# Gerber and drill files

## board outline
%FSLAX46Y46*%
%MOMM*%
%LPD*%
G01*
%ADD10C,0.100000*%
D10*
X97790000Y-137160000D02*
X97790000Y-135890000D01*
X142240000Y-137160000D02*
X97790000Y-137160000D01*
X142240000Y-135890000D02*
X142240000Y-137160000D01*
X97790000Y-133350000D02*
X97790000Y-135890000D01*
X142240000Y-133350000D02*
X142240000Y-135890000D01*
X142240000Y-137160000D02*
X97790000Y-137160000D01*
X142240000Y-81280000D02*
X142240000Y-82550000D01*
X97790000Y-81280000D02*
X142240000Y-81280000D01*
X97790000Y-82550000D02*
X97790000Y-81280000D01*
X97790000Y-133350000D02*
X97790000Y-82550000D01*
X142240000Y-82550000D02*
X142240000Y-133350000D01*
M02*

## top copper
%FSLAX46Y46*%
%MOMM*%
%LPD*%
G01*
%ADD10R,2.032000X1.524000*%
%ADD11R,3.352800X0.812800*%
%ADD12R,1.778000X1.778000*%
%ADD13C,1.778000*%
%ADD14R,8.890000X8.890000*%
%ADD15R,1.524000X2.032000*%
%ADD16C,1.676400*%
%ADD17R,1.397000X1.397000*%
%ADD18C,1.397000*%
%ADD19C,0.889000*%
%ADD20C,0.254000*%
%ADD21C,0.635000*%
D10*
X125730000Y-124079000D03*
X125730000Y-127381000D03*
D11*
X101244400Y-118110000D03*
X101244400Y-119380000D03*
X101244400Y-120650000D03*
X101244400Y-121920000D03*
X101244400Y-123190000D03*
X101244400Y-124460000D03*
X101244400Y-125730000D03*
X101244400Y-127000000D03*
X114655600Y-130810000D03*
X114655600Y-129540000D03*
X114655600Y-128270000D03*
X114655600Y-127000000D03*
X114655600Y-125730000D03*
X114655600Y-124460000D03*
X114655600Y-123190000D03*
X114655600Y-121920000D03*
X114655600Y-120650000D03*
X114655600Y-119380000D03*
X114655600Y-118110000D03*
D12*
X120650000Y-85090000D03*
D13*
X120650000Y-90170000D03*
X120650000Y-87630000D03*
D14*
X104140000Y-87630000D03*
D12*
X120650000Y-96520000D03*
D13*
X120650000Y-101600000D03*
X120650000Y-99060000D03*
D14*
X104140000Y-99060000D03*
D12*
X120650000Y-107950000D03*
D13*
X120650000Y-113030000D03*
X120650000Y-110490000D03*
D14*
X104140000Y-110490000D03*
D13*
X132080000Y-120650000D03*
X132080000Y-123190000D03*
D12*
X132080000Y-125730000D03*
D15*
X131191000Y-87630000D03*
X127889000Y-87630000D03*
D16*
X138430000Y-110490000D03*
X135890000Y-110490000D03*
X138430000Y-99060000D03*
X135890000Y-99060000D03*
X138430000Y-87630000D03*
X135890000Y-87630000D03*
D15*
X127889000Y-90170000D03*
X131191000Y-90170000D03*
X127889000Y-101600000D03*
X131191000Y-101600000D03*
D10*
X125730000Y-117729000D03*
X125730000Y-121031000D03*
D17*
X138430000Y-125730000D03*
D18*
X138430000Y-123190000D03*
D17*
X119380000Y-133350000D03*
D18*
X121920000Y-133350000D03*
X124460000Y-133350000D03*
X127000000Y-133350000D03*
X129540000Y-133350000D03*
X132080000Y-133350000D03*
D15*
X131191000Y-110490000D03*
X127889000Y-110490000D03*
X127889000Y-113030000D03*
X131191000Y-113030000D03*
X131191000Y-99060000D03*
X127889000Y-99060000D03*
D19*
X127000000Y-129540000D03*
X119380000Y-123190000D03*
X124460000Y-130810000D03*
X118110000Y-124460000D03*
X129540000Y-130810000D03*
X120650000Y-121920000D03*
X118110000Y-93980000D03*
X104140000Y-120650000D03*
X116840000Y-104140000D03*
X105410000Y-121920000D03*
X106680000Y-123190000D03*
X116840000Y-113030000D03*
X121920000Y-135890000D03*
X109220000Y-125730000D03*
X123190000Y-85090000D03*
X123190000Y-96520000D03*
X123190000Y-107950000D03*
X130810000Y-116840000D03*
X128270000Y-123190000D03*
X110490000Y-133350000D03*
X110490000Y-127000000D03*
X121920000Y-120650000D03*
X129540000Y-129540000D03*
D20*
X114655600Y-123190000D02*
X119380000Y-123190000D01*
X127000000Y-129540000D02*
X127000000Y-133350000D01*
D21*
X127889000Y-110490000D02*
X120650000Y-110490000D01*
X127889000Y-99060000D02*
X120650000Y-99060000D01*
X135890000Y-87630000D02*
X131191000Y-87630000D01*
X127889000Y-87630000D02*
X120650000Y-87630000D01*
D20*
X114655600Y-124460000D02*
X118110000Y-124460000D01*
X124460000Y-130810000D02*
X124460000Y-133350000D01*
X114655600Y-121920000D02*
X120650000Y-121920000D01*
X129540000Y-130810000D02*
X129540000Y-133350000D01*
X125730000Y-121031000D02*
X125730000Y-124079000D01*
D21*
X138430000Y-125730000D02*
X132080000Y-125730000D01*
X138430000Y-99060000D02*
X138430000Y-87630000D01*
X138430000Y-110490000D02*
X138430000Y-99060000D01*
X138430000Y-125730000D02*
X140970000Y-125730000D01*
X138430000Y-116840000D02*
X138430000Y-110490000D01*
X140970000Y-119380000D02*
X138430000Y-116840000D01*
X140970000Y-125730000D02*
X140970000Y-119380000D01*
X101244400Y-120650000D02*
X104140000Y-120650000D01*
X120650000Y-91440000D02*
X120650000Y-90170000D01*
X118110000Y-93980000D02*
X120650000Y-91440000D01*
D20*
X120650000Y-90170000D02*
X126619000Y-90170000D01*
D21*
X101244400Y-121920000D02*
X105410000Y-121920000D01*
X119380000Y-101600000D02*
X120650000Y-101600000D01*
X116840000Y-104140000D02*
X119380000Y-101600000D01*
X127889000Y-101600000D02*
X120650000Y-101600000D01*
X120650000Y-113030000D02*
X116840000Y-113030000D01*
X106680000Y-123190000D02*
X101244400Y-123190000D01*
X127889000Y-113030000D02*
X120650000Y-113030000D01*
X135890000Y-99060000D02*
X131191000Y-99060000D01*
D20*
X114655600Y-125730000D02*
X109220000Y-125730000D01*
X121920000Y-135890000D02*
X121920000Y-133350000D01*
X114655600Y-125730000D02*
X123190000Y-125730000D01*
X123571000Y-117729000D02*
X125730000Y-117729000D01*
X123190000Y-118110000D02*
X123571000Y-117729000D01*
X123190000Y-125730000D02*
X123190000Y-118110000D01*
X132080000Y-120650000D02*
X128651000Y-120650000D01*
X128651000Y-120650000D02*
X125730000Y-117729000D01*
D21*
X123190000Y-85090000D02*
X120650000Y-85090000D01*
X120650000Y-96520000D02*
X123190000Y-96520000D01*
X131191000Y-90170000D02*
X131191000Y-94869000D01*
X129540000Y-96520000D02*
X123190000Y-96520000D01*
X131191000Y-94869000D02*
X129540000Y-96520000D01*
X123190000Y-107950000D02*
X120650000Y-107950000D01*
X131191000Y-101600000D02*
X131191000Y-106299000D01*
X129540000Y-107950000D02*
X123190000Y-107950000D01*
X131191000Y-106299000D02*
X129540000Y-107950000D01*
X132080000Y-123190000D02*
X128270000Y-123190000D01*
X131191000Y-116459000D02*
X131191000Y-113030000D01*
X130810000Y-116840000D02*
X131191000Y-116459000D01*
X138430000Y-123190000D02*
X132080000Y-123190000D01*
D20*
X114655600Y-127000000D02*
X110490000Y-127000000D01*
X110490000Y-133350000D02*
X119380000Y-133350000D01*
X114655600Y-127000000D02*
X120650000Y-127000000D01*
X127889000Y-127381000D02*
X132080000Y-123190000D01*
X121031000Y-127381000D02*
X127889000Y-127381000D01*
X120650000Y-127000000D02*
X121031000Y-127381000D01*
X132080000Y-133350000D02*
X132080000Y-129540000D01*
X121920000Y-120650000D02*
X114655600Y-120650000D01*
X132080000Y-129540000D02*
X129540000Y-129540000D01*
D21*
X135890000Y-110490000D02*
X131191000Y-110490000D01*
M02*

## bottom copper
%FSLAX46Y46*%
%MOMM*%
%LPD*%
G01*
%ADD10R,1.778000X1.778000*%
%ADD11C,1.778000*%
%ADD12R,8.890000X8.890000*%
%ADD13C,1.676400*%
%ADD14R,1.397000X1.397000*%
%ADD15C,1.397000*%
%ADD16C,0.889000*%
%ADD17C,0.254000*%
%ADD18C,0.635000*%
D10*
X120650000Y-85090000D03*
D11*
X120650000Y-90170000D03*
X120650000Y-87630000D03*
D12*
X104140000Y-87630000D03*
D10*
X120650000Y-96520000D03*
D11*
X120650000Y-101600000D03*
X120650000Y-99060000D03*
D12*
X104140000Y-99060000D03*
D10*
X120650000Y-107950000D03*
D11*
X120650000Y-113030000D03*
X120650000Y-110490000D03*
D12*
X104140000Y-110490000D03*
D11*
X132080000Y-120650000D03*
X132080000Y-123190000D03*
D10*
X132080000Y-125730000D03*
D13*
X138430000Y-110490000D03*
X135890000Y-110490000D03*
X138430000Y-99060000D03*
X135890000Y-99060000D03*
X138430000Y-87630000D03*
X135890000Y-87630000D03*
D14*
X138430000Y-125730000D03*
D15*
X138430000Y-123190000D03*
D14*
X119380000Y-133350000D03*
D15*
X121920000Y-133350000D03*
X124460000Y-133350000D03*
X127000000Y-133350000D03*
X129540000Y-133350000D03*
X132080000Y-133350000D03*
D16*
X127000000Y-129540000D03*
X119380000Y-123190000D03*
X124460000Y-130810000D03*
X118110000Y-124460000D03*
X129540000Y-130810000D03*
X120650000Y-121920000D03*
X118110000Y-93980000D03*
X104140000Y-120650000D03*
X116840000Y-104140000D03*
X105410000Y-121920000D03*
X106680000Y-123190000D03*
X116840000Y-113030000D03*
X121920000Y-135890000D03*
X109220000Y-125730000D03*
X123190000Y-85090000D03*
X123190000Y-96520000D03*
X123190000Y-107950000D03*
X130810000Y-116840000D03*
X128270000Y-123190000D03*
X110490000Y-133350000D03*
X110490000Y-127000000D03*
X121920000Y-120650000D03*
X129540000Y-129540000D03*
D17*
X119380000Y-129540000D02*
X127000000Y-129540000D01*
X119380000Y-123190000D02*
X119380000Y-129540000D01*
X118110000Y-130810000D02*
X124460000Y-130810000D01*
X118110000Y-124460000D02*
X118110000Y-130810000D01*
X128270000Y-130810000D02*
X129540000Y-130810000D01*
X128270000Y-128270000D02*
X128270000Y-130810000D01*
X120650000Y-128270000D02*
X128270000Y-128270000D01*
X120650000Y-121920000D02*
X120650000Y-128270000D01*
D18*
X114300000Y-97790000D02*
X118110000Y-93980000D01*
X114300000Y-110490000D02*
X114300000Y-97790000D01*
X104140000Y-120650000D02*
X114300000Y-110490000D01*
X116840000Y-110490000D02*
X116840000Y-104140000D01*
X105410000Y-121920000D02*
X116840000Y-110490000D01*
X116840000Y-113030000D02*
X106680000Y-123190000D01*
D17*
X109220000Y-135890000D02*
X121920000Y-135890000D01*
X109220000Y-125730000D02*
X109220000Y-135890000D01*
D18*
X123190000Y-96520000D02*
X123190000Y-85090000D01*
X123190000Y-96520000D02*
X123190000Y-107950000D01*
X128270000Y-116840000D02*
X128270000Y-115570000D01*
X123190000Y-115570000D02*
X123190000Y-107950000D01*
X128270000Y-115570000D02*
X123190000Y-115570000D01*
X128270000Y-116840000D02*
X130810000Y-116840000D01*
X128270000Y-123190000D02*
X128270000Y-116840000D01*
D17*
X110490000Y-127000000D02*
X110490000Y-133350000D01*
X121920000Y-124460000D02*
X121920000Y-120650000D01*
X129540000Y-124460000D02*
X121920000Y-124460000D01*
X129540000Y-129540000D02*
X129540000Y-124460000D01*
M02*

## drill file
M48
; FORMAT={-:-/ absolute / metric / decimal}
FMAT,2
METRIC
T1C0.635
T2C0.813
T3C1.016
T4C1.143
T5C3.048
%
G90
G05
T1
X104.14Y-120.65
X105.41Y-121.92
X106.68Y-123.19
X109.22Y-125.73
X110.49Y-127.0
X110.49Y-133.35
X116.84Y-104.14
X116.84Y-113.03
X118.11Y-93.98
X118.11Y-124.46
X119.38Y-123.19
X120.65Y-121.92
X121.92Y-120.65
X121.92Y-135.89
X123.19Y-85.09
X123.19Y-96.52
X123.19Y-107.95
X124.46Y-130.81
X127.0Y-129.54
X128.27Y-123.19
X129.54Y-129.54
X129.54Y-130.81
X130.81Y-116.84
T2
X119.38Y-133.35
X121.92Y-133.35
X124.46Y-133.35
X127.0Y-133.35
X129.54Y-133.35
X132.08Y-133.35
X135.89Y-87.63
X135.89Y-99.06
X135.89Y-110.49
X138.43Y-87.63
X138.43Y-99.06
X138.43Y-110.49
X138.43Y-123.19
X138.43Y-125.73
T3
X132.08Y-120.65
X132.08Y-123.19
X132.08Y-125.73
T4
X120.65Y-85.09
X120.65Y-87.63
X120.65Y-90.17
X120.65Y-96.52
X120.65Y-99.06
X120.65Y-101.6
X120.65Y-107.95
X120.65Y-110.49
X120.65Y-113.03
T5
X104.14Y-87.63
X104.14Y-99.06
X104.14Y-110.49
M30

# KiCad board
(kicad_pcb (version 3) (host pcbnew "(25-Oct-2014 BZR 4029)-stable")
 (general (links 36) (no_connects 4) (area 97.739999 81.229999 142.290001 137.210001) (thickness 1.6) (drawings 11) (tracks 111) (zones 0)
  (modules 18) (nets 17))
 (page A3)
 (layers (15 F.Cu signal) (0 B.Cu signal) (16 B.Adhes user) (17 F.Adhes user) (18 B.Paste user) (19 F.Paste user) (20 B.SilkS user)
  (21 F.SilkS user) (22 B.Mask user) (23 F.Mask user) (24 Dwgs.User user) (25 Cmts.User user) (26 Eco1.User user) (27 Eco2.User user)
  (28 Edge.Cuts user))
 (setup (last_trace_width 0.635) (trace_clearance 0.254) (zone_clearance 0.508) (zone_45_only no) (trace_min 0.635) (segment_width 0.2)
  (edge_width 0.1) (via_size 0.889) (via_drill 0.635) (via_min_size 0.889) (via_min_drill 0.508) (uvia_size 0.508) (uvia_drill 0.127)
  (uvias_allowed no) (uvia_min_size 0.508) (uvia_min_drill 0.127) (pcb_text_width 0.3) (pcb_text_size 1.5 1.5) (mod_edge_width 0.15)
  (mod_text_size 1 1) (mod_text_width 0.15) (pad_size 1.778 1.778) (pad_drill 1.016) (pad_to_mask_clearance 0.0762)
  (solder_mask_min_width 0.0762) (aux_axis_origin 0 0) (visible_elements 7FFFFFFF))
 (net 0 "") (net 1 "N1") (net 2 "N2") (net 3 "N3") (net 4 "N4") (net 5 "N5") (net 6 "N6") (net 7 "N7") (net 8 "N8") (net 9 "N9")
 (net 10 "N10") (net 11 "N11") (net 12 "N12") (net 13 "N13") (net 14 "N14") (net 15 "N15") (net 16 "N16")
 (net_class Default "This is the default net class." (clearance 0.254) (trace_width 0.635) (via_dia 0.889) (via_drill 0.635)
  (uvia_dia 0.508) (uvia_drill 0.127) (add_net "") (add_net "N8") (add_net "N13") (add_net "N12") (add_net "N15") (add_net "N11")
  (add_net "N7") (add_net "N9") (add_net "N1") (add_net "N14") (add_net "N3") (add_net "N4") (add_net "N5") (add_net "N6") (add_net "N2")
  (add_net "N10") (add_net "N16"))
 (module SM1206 (layer F.Cu) (at 125.73 125.73 270)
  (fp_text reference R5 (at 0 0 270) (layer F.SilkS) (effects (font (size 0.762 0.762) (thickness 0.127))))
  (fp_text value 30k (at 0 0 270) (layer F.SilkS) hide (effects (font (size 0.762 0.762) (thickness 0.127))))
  (pad 1 smd rect (at -1.651 0 270) (size 1.524 2.032) (layers F.Cu F.Paste F.Mask) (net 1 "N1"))
  (pad 2 smd rect (at 1.651 0 270) (size 1.524 2.032) (layers F.Cu F.Paste F.Mask) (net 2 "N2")))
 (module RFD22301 (layer F.Cu) (at 106.68 125.73)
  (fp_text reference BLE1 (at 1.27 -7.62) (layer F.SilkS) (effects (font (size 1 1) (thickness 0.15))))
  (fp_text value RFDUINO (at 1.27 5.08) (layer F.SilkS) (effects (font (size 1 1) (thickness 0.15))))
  (pad 1 smd rect (at -5.4356 -7.62) (size 3.3528 0.8128) (layers F.Cu F.Paste F.Mask))
  (pad 2 smd rect (at -5.4356 -6.35) (size 3.3528 0.8128) (layers F.Cu F.Paste F.Mask))
  (pad 3 smd rect (at -5.4356 -5.08) (size 3.3528 0.8128) (layers F.Cu F.Paste F.Mask) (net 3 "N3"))
  (pad 4 smd rect (at -5.4356 -3.81) (size 3.3528 0.8128) (layers F.Cu F.Paste F.Mask) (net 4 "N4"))
  (pad 5 smd rect (at -5.4356 -2.54) (size 3.3528 0.8128) (layers F.Cu F.Paste F.Mask) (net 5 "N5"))
  (pad 6 smd rect (at -5.4356 -1.27) (size 3.3528 0.8128) (layers F.Cu F.Paste F.Mask) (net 1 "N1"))
  (pad 7 smd rect (at -5.4356 0) (size 3.3528 0.8128) (layers F.Cu F.Paste F.Mask))
  (pad 8 smd rect (at -5.4356 1.27) (size 3.3528 0.8128) (layers F.Cu F.Paste F.Mask))
  (pad 9 smd rect (at 7.9756 5.08) (size 3.3528 0.8128) (layers F.Cu F.Paste F.Mask))
  (pad 10 smd rect (at 7.9756 3.81) (size 3.3528 0.8128) (layers F.Cu F.Paste F.Mask))
  (pad 11 smd rect (at 7.9756 2.54) (size 3.3528 0.8128) (layers F.Cu F.Paste F.Mask))
  (pad 12 smd rect (at 7.9756 1.27) (size 3.3528 0.8128) (layers F.Cu F.Paste F.Mask) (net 2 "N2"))
  (pad 13 smd rect (at 7.9756 0) (size 3.3528 0.8128) (layers F.Cu F.Paste F.Mask) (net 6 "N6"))
  (pad 14 smd rect (at 7.9756 -1.27) (size 3.3528 0.8128) (layers F.Cu F.Paste F.Mask) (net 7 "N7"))
  (pad 15 smd rect (at 7.9756 -2.54) (size 3.3528 0.8128) (layers F.Cu F.Paste F.Mask) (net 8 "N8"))
  (pad 16 smd rect (at 7.9756 -3.81) (size 3.3528 0.8128) (layers F.Cu F.Paste F.Mask) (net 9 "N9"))
  (pad 17 smd rect (at 7.9756 -5.08) (size 3.3528 0.8128) (layers F.Cu F.Paste F.Mask) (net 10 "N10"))
  (pad 18 smd rect (at 7.9756 -6.35) (size 3.3528 0.8128) (layers F.Cu F.Paste F.Mask))
  (pad 19 smd rect (at 7.9756 -7.62) (size 3.3528 0.8128) (layers F.Cu F.Paste F.Mask)))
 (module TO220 (layer F.Cu) (at 120.65 87.63 180)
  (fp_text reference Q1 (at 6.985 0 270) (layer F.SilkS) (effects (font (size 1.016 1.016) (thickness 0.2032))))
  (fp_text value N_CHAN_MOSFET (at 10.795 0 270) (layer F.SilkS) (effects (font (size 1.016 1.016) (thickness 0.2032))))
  (pad 1 thru_hole rect (at 0 2.54 180) (size 1.778 1.778) (drill 1.143) (layers *.Cu *.Mask F.SilkS) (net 2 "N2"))
  (pad 2 thru_hole circle (at 0 -2.54 180) (size 1.778 1.778) (drill 1.143) (layers *.Cu *.Mask F.SilkS) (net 3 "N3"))
  (pad 3 thru_hole circle (at 0 0 180) (size 1.778 1.778) (drill 1.143) (layers *.Cu *.Mask F.SilkS) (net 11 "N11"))
  (pad 4 thru_hole rect (at 16.51 0 180) (size 8.89 8.89) (drill 3.048) (layers *.Cu *.SilkS *.Mask)))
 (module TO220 (layer F.Cu) (at 120.65 99.06 180)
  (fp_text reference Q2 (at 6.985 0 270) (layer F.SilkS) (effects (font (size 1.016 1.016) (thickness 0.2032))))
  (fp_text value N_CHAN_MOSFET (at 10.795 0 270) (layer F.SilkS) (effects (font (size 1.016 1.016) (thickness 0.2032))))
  (pad 1 thru_hole rect (at 0 2.54 180) (size 1.778 1.778) (drill 1.143) (layers *.Cu *.Mask F.SilkS) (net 2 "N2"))
  (pad 2 thru_hole circle (at 0 -2.54 180) (size 1.778 1.778) (drill 1.143) (layers *.Cu *.Mask F.SilkS) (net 4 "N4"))
  (pad 3 thru_hole circle (at 0 0 180) (size 1.778 1.778) (drill 1.143) (layers *.Cu *.Mask F.SilkS) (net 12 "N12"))
  (pad 4 thru_hole rect (at 16.51 0 180) (size 8.89 8.89) (drill 3.048) (layers *.Cu *.SilkS *.Mask)))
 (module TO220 (layer F.Cu) (at 120.65 110.49 180)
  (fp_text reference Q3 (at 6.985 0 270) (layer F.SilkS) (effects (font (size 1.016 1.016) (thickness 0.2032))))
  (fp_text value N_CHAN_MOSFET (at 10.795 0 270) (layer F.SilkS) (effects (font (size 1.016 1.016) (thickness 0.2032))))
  (pad 1 thru_hole rect (at 0 2.54 180) (size 1.778 1.778) (drill 1.143) (layers *.Cu *.Mask F.SilkS) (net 2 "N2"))
  (pad 2 thru_hole circle (at 0 -2.54 180) (size 1.778 1.778) (drill 1.143) (layers *.Cu *.Mask F.SilkS) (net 5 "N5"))
  (pad 3 thru_hole circle (at 0 0 180) (size 1.778 1.778) (drill 1.143) (layers *.Cu *.Mask F.SilkS) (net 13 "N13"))
  (pad 4 thru_hole rect (at 16.51 0 180) (size 8.89 8.89) (drill 3.048) (layers *.Cu *.SilkS *.Mask)))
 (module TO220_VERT (layer F.Cu) (at 132.08 123.19)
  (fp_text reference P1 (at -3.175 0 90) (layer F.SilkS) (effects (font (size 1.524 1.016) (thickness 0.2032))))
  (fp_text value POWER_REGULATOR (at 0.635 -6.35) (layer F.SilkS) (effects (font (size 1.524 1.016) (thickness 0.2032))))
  (pad 2 thru_hole circle (at 0 -2.54) (size 1.778 1.778) (drill 1.016) (layers *.Cu *.Mask F.SilkS) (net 6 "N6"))
  (pad 3 thru_hole circle (at 0 0) (size 1.778 1.778) (drill 1.016) (layers *.Cu *.Mask F.SilkS) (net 2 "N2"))
  (pad 1 thru_hole rect (at 0 2.54) (size 1.778 1.778) (drill 1.016) (layers *.Cu *.Mask F.SilkS) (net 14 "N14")))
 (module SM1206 (layer F.Cu) (at 129.54 87.63 180)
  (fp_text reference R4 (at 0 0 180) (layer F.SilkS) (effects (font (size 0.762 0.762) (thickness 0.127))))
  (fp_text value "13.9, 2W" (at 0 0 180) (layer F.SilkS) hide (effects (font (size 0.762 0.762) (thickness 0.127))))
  (pad 1 smd rect (at -1.651 0 180) (size 1.524 2.032) (layers F.Cu F.Paste F.Mask) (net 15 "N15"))
  (pad 2 smd rect (at 1.651 0 180) (size 1.524 2.032) (layers F.Cu F.Paste F.Mask) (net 11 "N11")))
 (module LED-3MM (layer F.Cu) (at 137.16 110.49 180)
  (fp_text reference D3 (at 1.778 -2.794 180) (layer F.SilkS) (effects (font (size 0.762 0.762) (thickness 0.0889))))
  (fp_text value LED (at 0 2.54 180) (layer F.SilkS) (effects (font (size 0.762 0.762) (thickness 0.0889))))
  (pad 1 thru_hole circle (at -1.27 0 180) (size 1.6764 1.6764) (drill 0.8128) (layers *.Cu *.Mask F.SilkS) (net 14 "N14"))
  (pad 2 thru_hole circle (at 1.27 0 180) (size 1.6764 1.6764) (drill 0.8128) (layers *.Cu *.Mask F.SilkS) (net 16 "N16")))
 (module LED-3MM (layer F.Cu) (at 137.16 99.06 180)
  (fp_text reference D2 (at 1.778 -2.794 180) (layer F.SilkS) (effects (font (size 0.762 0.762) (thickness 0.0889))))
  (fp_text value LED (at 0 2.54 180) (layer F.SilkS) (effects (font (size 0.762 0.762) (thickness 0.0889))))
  (pad 1 thru_hole circle (at -1.27 0 180) (size 1.6764 1.6764) (drill 0.8128) (layers *.Cu *.Mask F.SilkS) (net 14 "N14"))
  (pad 2 thru_hole circle (at 1.27 0 180) (size 1.6764 1.6764) (drill 0.8128) (layers *.Cu *.Mask F.SilkS) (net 5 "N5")))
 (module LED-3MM (layer F.Cu) (at 137.16 87.63 180)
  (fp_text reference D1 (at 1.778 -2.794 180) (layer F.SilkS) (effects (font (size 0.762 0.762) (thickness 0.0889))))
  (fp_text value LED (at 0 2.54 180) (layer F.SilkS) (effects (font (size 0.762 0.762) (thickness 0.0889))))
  (pad 1 thru_hole circle (at -1.27 0 180) (size 1.6764 1.6764) (drill 0.8128) (layers *.Cu *.Mask F.SilkS) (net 14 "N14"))
  (pad 2 thru_hole circle (at 1.27 0 180) (size 1.6764 1.6764) (drill 0.8128) (layers *.Cu *.Mask F.SilkS) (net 15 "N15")))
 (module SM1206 (layer F.Cu) (at 129.54 90.17)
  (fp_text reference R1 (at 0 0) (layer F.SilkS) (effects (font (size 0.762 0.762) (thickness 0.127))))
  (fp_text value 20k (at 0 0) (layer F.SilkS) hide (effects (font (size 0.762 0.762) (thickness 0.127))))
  (pad 1 smd rect (at -1.651 0) (size 1.524 2.032) (layers F.Cu F.Paste F.Mask) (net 3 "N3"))
  (pad 2 smd rect (at 1.651 0) (size 1.524 2.032) (layers F.Cu F.Paste F.Mask) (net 2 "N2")))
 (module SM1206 (layer F.Cu) (at 129.54 101.6)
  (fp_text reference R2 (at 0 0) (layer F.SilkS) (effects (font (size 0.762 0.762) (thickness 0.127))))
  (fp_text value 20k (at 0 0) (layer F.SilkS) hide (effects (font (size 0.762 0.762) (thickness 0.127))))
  (pad 1 smd rect (at -1.651 0) (size 1.524 2.032) (layers F.Cu F.Paste F.Mask) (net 4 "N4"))
  (pad 2 smd rect (at 1.651 0) (size 1.524 2.032) (layers F.Cu F.Paste F.Mask) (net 2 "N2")))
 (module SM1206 (layer F.Cu) (at 125.73 119.38 270)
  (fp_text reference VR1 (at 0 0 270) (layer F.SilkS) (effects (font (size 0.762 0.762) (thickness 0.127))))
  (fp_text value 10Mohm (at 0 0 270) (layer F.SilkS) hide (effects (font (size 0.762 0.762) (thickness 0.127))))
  (pad 1 smd rect (at -1.651 0 270) (size 1.524 2.032) (layers F.Cu F.Paste F.Mask) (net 6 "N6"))
  (pad 2 smd rect (at 1.651 0 270) (size 1.524 2.032) (layers F.Cu F.Paste F.Mask) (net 1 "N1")))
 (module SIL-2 (layer F.Cu) (at 138.43 124.46 90)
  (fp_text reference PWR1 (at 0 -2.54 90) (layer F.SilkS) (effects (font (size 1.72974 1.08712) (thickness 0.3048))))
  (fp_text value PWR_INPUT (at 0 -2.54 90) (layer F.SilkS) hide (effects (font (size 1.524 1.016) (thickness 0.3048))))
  (pad 1 thru_hole rect (at -1.27 0 90) (size 1.397 1.397) (drill 0.8128) (layers *.Cu *.Mask F.SilkS) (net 14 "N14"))
  (pad 2 thru_hole circle (at 1.27 0 90) (size 1.397 1.397) (drill 0.8128) (layers *.Cu *.Mask F.SilkS) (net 2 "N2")))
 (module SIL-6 (layer F.Cu) (at 125.73 133.35)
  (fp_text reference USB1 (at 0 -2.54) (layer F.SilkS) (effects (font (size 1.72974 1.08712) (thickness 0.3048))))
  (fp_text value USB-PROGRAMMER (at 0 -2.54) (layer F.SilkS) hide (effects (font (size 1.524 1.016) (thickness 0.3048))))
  (pad 1 thru_hole rect (at -6.35 0) (size 1.397 1.397) (drill 0.8128) (layers *.Cu *.Mask F.SilkS) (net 2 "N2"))
  (pad 2 thru_hole circle (at -3.81 0) (size 1.397 1.397) (drill 0.8128) (layers *.Cu *.Mask F.SilkS) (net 6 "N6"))
  (pad 3 thru_hole circle (at -1.27 0) (size 1.397 1.397) (drill 0.8128) (layers *.Cu *.Mask F.SilkS) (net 7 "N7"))
  (pad 4 thru_hole circle (at 1.27 0) (size 1.397 1.397) (drill 0.8128) (layers *.Cu *.Mask F.SilkS) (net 8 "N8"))
  (pad 5 thru_hole circle (at 3.81 0) (size 1.397 1.397) (drill 0.8128) (layers *.Cu *.Mask F.SilkS) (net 9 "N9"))
  (pad 6 thru_hole circle (at 6.35 0) (size 1.397 1.397) (drill 0.8128) (layers *.Cu *.Mask F.SilkS) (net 10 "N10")))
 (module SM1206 (layer F.Cu) (at 129.54 110.49 180)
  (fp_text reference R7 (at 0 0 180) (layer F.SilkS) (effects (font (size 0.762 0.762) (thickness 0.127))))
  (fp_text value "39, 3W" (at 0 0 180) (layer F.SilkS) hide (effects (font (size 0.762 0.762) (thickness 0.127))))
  (pad 1 smd rect (at -1.651 0 180) (size 1.524 2.032) (layers F.Cu F.Paste F.Mask) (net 16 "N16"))
  (pad 2 smd rect (at 1.651 0 180) (size 1.524 2.032) (layers F.Cu F.Paste F.Mask) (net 13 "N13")))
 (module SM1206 (layer F.Cu) (at 129.54 113.03)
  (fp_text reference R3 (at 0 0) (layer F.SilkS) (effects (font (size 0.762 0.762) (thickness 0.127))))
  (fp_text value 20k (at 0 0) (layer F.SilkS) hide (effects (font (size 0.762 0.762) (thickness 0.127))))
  (pad 1 smd rect (at -1.651 0) (size 1.524 2.032) (layers F.Cu F.Paste F.Mask) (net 5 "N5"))
  (pad 2 smd rect (at 1.651 0) (size 1.524 2.032) (layers F.Cu F.Paste F.Mask) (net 2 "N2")))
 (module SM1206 (layer F.Cu) (at 129.54 99.06 180)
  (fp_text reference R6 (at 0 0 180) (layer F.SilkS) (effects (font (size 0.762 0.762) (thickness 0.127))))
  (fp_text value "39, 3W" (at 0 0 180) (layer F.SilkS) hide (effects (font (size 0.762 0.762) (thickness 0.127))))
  (pad 1 smd rect (at -1.651 0 180) (size 1.524 2.032) (layers F.Cu F.Paste F.Mask) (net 5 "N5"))
  (pad 2 smd rect (at 1.651 0 180) (size 1.524 2.032) (layers F.Cu F.Paste F.Mask) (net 12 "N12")))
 (gr_line (start 97.79 137.16) (end 97.79 135.89) (angle 90) (layer Edge.Cuts) (width 0.1))
 (gr_line (start 142.24 137.16) (end 97.79 137.16) (angle 90) (layer Edge.Cuts) (width 0.1))
 (gr_line (start 142.24 135.89) (end 142.24 137.16) (angle 90) (layer Edge.Cuts) (width 0.1))
 (gr_line (start 97.79 133.35) (end 97.79 135.89) (angle 90) (layer Edge.Cuts) (width 0.1))
 (gr_line (start 142.24 133.35) (end 142.24 135.89) (angle 90) (layer Edge.Cuts) (width 0.1))
 (gr_line (start 142.24 137.16) (end 97.79 137.16) (angle 90) (layer Edge.Cuts) (width 0.1))
 (gr_line (start 142.24 81.28) (end 142.24 82.55) (angle 90) (layer Edge.Cuts) (width 0.1))
 (gr_line (start 97.79 81.28) (end 142.24 81.28) (angle 90) (layer Edge.Cuts) (width 0.1))
 (gr_line (start 97.79 82.55) (end 97.79 81.28) (angle 90) (layer Edge.Cuts) (width 0.1))
 (gr_line (start 97.79 133.35) (end 97.79 82.55) (angle 90) (layer Edge.Cuts) (width 0.1))
 (gr_line (start 142.24 82.55) (end 142.24 133.35) (angle 90) (layer Edge.Cuts) (width 0.1))
 (segment (start 114.6556 123.19) (end 119.38 123.19) (width 0.254) (layer F.Cu) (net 8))
 (segment (start 127 129.54) (end 127 133.35) (width 0.254) (layer F.Cu) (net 8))
 (via (at 127 129.54) (size 0.889) (layers F.Cu B.Cu) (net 8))
 (segment (start 119.38 129.54) (end 127 129.54) (width 0.254) (layer B.Cu) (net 8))
 (segment (start 119.38 123.19) (end 119.38 129.54) (width 0.254) (layer B.Cu) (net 8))
 (via (at 119.38 123.19) (size 0.889) (layers F.Cu B.Cu) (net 8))
 (segment (start 127.889 110.49) (end 120.65 110.49) (width 0.635) (layer F.Cu) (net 13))
 (segment (start 127.889 99.06) (end 120.65 99.06) (width 0.635) (layer F.Cu) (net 12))
 (segment (start 135.89 87.63) (end 131.191 87.63) (width 0.635) (layer F.Cu) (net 15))
 (segment (start 127.889 87.63) (end 120.65 87.63) (width 0.635) (layer F.Cu) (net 11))
 (segment (start 114.6556 124.46) (end 118.11 124.46) (width 0.254) (layer F.Cu) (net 7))
 (segment (start 124.46 130.81) (end 124.46 133.35) (width 0.254) (layer F.Cu) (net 7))
 (via (at 124.46 130.81) (size 0.889) (layers F.Cu B.Cu) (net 7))
 (segment (start 118.11 130.81) (end 124.46 130.81) (width 0.254) (layer B.Cu) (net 7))
 (segment (start 118.11 124.46) (end 118.11 130.81) (width 0.254) (layer B.Cu) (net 7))
 (via (at 118.11 124.46) (size 0.889) (layers F.Cu B.Cu) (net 7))
 (segment (start 114.6556 121.92) (end 120.65 121.92) (width 0.254) (layer F.Cu) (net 9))
 (segment (start 129.54 130.81) (end 129.54 133.35) (width 0.254) (layer F.Cu) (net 9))
 (via (at 129.54 130.81) (size 0.889) (layers F.Cu B.Cu) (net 9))
 (segment (start 128.27 130.81) (end 129.54 130.81) (width 0.254) (layer B.Cu) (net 9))
 (segment (start 128.27 128.27) (end 128.27 130.81) (width 0.254) (layer B.Cu) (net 9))
 (segment (start 120.65 128.27) (end 128.27 128.27) (width 0.254) (layer B.Cu) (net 9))
 (segment (start 120.65 121.92) (end 120.65 128.27) (width 0.254) (layer B.Cu) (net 9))
 (via (at 120.65 121.92) (size 0.889) (layers F.Cu B.Cu) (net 9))
 (segment (start 125.73 121.031) (end 125.73 124.079) (width 0.254) (layer F.Cu) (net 1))
 (segment (start 138.43 125.73) (end 132.08 125.73) (width 0.635) (layer F.Cu) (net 14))
 (segment (start 138.43 99.06) (end 138.43 87.63) (width 0.635) (layer F.Cu) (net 14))
 (segment (start 138.43 110.49) (end 138.43 99.06) (width 0.635) (layer F.Cu) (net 14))
 (segment (start 138.43 125.73) (end 140.97 125.73) (width 0.635) (layer F.Cu) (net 14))
 (segment (start 138.43 116.84) (end 138.43 110.49) (width 0.635) (layer F.Cu) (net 14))
 (segment (start 140.97 119.38) (end 138.43 116.84) (width 0.635) (layer F.Cu) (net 14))
 (segment (start 140.97 125.73) (end 140.97 119.38) (width 0.635) (layer F.Cu) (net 14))
 (segment (start 101.2444 120.65) (end 104.14 120.65) (width 0.635) (layer F.Cu) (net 3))
 (segment (start 120.65 91.44) (end 120.65 90.17) (width 0.635) (layer F.Cu) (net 3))
 (segment (start 118.11 93.98) (end 120.65 91.44) (width 0.635) (layer F.Cu) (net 3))
 (via (at 118.11 93.98) (size 0.889) (layers F.Cu B.Cu) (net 3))
 (segment (start 114.3 97.79) (end 118.11 93.98) (width 0.635) (layer B.Cu) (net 3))
 (segment (start 114.3 110.49) (end 114.3 97.79) (width 0.635) (layer B.Cu) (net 3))
 (segment (start 104.14 120.65) (end 114.3 110.49) (width 0.635) (layer B.Cu) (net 3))
 (via (at 104.14 120.65) (size 0.889) (layers F.Cu B.Cu) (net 3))
 (segment (start 120.65 90.17) (end 126.619 90.17) (width 0.254) (layer F.Cu) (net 3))
 (segment (start 101.2444 121.92) (end 105.41 121.92) (width 0.635) (layer F.Cu) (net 4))
 (segment (start 119.38 101.6) (end 120.65 101.6) (width 0.635) (layer F.Cu) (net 4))
 (segment (start 116.84 104.14) (end 119.38 101.6) (width 0.635) (layer F.Cu) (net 4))
 (via (at 116.84 104.14) (size 0.889) (layers F.Cu B.Cu) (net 4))
 (segment (start 116.84 110.49) (end 116.84 104.14) (width 0.635) (layer B.Cu) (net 4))
 (segment (start 105.41 121.92) (end 116.84 110.49) (width 0.635) (layer B.Cu) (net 4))
 (via (at 105.41 121.92) (size 0.889) (layers F.Cu B.Cu) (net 4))
 (segment (start 127.889 101.6) (end 120.65 101.6) (width 0.635) (layer F.Cu) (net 4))
 (segment (start 120.65 113.03) (end 116.84 113.03) (width 0.635) (layer F.Cu) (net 5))
 (segment (start 106.68 123.19) (end 101.2444 123.19) (width 0.635) (layer F.Cu) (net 5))
 (via (at 106.68 123.19) (size 0.889) (layers F.Cu B.Cu) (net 5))
 (segment (start 116.84 113.03) (end 106.68 123.19) (width 0.635) (layer B.Cu) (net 5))
 (via (at 116.84 113.03) (size 0.889) (layers F.Cu B.Cu) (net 5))
 (segment (start 127.889 113.03) (end 120.65 113.03) (width 0.635) (layer F.Cu) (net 5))
 (segment (start 135.89 99.06) (end 131.191 99.06) (width 0.635) (layer F.Cu) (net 5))
 (segment (start 114.6556 125.73) (end 109.22 125.73) (width 0.254) (layer F.Cu) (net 6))
 (segment (start 121.92 135.89) (end 121.92 133.35) (width 0.254) (layer F.Cu) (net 6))
 (via (at 121.92 135.89) (size 0.889) (layers F.Cu B.Cu) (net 6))
 (segment (start 109.22 135.89) (end 121.92 135.89) (width 0.254) (layer B.Cu) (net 6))
 (segment (start 109.22 125.73) (end 109.22 135.89) (width 0.254) (layer B.Cu) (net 6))
 (via (at 109.22 125.73) (size 0.889) (layers F.Cu B.Cu) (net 6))
 (segment (start 114.6556 125.73) (end 123.19 125.73) (width 0.254) (layer F.Cu) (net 6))
 (segment (start 123.571 117.729) (end 125.73 117.729) (width 0.254) (layer F.Cu) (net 6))
 (segment (start 123.19 118.11) (end 123.571 117.729) (width 0.254) (layer F.Cu) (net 6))
 (segment (start 123.19 125.73) (end 123.19 118.11) (width 0.254) (layer F.Cu) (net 6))
 (segment (start 132.08 120.65) (end 128.651 120.65) (width 0.254) (layer F.Cu) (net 6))
 (segment (start 128.651 120.65) (end 125.73 117.729) (width 0.254) (layer F.Cu) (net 6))
 (segment (start 123.19 96.52) (end 123.19 85.09) (width 0.635) (layer B.Cu) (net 2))
 (segment (start 123.19 85.09) (end 120.65 85.09) (width 0.635) (layer F.Cu) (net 2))
 (via (at 123.19 85.09) (size 0.889) (layers F.Cu B.Cu) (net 2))
 (segment (start 120.65 96.52) (end 123.19 96.52) (width 0.635) (layer F.Cu) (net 2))
 (segment (start 131.191 90.17) (end 131.191 94.869) (width 0.635) (layer F.Cu) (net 2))
 (segment (start 123.19 96.52) (end 123.19 107.95) (width 0.635) (layer B.Cu) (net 2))
 (via (at 123.19 96.52) (size 0.889) (layers F.Cu B.Cu) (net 2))
 (segment (start 129.54 96.52) (end 123.19 96.52) (width 0.635) (layer F.Cu) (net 2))
 (segment (start 131.191 94.869) (end 129.54 96.52) (width 0.635) (layer F.Cu) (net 2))
 (segment (start 123.19 107.95) (end 120.65 107.95) (width 0.635) (layer F.Cu) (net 2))
 (segment (start 131.191 101.6) (end 131.191 106.299) (width 0.635) (layer F.Cu) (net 2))
 (segment (start 129.54 107.95) (end 123.19 107.95) (width 0.635) (layer F.Cu) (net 2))
 (segment (start 131.191 106.299) (end 129.54 107.95) (width 0.635) (layer F.Cu) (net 2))
 (segment (start 128.27 116.84) (end 128.27 115.57) (width 0.635) (layer B.Cu) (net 2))
 (via (at 123.19 107.95) (size 0.889) (layers F.Cu B.Cu) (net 2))
 (segment (start 123.19 115.57) (end 123.19 107.95) (width 0.635) (layer B.Cu) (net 2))
 (segment (start 128.27 115.57) (end 123.19 115.57) (width 0.635) (layer B.Cu) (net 2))
 (segment (start 132.08 123.19) (end 128.27 123.19) (width 0.635) (layer F.Cu) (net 2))
 (segment (start 131.191 116.459) (end 131.191 113.03) (width 0.635) (layer F.Cu) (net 2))
 (segment (start 130.81 116.84) (end 131.191 116.459) (width 0.635) (layer F.Cu) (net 2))
 (via (at 130.81 116.84) (size 0.889) (layers F.Cu B.Cu) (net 2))
 (segment (start 128.27 116.84) (end 130.81 116.84) (width 0.635) (layer B.Cu) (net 2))
 (segment (start 128.27 123.19) (end 128.27 116.84) (width 0.635) (layer B.Cu) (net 2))
 (via (at 128.27 123.19) (size 0.889) (layers F.Cu B.Cu) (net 2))
 (segment (start 138.43 123.19) (end 132.08 123.19) (width 0.635) (layer F.Cu) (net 2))
 (segment (start 114.6556 127) (end 110.49 127) (width 0.254) (layer F.Cu) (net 2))
 (segment (start 110.49 133.35) (end 119.38 133.35) (width 0.254) (layer F.Cu) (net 2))
 (via (at 110.49 133.35) (size 0.889) (layers F.Cu B.Cu) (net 2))
 (segment (start 110.49 127) (end 110.49 133.35) (width 0.254) (layer B.Cu) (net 2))
 (via (at 110.49 127) (size 0.889) (layers F.Cu B.Cu) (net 2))
 (segment (start 114.6556 127) (end 120.65 127) (width 0.254) (layer F.Cu) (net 2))
 (segment (start 127.889 127.381) (end 132.08 123.19) (width 0.254) (layer F.Cu) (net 2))
 (segment (start 121.031 127.381) (end 127.889 127.381) (width 0.254) (layer F.Cu) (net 2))
 (segment (start 120.65 127) (end 121.031 127.381) (width 0.254) (layer F.Cu) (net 2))
 (segment (start 132.08 133.35) (end 132.08 129.54) (width 0.254) (layer F.Cu) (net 10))
 (segment (start 121.92 120.65) (end 114.6556 120.65) (width 0.254) (layer F.Cu) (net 10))
 (via (at 121.92 120.65) (size 0.889) (layers F.Cu B.Cu) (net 10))
 (segment (start 121.92 124.46) (end 121.92 120.65) (width 0.254) (layer B.Cu) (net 10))
 (segment (start 129.54 124.46) (end 121.92 124.46) (width 0.254) (layer B.Cu) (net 10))
 (segment (start 129.54 129.54) (end 129.54 124.46) (width 0.254) (layer B.Cu) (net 10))
 (via (at 129.54 129.54) (size 0.889) (layers F.Cu B.Cu) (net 10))
 (segment (start 132.08 129.54) (end 129.54 129.54) (width 0.254) (layer F.Cu) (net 10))
 (segment (start 135.89 110.49) (end 131.191 110.49) (width 0.635) (layer F.Cu) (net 16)))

